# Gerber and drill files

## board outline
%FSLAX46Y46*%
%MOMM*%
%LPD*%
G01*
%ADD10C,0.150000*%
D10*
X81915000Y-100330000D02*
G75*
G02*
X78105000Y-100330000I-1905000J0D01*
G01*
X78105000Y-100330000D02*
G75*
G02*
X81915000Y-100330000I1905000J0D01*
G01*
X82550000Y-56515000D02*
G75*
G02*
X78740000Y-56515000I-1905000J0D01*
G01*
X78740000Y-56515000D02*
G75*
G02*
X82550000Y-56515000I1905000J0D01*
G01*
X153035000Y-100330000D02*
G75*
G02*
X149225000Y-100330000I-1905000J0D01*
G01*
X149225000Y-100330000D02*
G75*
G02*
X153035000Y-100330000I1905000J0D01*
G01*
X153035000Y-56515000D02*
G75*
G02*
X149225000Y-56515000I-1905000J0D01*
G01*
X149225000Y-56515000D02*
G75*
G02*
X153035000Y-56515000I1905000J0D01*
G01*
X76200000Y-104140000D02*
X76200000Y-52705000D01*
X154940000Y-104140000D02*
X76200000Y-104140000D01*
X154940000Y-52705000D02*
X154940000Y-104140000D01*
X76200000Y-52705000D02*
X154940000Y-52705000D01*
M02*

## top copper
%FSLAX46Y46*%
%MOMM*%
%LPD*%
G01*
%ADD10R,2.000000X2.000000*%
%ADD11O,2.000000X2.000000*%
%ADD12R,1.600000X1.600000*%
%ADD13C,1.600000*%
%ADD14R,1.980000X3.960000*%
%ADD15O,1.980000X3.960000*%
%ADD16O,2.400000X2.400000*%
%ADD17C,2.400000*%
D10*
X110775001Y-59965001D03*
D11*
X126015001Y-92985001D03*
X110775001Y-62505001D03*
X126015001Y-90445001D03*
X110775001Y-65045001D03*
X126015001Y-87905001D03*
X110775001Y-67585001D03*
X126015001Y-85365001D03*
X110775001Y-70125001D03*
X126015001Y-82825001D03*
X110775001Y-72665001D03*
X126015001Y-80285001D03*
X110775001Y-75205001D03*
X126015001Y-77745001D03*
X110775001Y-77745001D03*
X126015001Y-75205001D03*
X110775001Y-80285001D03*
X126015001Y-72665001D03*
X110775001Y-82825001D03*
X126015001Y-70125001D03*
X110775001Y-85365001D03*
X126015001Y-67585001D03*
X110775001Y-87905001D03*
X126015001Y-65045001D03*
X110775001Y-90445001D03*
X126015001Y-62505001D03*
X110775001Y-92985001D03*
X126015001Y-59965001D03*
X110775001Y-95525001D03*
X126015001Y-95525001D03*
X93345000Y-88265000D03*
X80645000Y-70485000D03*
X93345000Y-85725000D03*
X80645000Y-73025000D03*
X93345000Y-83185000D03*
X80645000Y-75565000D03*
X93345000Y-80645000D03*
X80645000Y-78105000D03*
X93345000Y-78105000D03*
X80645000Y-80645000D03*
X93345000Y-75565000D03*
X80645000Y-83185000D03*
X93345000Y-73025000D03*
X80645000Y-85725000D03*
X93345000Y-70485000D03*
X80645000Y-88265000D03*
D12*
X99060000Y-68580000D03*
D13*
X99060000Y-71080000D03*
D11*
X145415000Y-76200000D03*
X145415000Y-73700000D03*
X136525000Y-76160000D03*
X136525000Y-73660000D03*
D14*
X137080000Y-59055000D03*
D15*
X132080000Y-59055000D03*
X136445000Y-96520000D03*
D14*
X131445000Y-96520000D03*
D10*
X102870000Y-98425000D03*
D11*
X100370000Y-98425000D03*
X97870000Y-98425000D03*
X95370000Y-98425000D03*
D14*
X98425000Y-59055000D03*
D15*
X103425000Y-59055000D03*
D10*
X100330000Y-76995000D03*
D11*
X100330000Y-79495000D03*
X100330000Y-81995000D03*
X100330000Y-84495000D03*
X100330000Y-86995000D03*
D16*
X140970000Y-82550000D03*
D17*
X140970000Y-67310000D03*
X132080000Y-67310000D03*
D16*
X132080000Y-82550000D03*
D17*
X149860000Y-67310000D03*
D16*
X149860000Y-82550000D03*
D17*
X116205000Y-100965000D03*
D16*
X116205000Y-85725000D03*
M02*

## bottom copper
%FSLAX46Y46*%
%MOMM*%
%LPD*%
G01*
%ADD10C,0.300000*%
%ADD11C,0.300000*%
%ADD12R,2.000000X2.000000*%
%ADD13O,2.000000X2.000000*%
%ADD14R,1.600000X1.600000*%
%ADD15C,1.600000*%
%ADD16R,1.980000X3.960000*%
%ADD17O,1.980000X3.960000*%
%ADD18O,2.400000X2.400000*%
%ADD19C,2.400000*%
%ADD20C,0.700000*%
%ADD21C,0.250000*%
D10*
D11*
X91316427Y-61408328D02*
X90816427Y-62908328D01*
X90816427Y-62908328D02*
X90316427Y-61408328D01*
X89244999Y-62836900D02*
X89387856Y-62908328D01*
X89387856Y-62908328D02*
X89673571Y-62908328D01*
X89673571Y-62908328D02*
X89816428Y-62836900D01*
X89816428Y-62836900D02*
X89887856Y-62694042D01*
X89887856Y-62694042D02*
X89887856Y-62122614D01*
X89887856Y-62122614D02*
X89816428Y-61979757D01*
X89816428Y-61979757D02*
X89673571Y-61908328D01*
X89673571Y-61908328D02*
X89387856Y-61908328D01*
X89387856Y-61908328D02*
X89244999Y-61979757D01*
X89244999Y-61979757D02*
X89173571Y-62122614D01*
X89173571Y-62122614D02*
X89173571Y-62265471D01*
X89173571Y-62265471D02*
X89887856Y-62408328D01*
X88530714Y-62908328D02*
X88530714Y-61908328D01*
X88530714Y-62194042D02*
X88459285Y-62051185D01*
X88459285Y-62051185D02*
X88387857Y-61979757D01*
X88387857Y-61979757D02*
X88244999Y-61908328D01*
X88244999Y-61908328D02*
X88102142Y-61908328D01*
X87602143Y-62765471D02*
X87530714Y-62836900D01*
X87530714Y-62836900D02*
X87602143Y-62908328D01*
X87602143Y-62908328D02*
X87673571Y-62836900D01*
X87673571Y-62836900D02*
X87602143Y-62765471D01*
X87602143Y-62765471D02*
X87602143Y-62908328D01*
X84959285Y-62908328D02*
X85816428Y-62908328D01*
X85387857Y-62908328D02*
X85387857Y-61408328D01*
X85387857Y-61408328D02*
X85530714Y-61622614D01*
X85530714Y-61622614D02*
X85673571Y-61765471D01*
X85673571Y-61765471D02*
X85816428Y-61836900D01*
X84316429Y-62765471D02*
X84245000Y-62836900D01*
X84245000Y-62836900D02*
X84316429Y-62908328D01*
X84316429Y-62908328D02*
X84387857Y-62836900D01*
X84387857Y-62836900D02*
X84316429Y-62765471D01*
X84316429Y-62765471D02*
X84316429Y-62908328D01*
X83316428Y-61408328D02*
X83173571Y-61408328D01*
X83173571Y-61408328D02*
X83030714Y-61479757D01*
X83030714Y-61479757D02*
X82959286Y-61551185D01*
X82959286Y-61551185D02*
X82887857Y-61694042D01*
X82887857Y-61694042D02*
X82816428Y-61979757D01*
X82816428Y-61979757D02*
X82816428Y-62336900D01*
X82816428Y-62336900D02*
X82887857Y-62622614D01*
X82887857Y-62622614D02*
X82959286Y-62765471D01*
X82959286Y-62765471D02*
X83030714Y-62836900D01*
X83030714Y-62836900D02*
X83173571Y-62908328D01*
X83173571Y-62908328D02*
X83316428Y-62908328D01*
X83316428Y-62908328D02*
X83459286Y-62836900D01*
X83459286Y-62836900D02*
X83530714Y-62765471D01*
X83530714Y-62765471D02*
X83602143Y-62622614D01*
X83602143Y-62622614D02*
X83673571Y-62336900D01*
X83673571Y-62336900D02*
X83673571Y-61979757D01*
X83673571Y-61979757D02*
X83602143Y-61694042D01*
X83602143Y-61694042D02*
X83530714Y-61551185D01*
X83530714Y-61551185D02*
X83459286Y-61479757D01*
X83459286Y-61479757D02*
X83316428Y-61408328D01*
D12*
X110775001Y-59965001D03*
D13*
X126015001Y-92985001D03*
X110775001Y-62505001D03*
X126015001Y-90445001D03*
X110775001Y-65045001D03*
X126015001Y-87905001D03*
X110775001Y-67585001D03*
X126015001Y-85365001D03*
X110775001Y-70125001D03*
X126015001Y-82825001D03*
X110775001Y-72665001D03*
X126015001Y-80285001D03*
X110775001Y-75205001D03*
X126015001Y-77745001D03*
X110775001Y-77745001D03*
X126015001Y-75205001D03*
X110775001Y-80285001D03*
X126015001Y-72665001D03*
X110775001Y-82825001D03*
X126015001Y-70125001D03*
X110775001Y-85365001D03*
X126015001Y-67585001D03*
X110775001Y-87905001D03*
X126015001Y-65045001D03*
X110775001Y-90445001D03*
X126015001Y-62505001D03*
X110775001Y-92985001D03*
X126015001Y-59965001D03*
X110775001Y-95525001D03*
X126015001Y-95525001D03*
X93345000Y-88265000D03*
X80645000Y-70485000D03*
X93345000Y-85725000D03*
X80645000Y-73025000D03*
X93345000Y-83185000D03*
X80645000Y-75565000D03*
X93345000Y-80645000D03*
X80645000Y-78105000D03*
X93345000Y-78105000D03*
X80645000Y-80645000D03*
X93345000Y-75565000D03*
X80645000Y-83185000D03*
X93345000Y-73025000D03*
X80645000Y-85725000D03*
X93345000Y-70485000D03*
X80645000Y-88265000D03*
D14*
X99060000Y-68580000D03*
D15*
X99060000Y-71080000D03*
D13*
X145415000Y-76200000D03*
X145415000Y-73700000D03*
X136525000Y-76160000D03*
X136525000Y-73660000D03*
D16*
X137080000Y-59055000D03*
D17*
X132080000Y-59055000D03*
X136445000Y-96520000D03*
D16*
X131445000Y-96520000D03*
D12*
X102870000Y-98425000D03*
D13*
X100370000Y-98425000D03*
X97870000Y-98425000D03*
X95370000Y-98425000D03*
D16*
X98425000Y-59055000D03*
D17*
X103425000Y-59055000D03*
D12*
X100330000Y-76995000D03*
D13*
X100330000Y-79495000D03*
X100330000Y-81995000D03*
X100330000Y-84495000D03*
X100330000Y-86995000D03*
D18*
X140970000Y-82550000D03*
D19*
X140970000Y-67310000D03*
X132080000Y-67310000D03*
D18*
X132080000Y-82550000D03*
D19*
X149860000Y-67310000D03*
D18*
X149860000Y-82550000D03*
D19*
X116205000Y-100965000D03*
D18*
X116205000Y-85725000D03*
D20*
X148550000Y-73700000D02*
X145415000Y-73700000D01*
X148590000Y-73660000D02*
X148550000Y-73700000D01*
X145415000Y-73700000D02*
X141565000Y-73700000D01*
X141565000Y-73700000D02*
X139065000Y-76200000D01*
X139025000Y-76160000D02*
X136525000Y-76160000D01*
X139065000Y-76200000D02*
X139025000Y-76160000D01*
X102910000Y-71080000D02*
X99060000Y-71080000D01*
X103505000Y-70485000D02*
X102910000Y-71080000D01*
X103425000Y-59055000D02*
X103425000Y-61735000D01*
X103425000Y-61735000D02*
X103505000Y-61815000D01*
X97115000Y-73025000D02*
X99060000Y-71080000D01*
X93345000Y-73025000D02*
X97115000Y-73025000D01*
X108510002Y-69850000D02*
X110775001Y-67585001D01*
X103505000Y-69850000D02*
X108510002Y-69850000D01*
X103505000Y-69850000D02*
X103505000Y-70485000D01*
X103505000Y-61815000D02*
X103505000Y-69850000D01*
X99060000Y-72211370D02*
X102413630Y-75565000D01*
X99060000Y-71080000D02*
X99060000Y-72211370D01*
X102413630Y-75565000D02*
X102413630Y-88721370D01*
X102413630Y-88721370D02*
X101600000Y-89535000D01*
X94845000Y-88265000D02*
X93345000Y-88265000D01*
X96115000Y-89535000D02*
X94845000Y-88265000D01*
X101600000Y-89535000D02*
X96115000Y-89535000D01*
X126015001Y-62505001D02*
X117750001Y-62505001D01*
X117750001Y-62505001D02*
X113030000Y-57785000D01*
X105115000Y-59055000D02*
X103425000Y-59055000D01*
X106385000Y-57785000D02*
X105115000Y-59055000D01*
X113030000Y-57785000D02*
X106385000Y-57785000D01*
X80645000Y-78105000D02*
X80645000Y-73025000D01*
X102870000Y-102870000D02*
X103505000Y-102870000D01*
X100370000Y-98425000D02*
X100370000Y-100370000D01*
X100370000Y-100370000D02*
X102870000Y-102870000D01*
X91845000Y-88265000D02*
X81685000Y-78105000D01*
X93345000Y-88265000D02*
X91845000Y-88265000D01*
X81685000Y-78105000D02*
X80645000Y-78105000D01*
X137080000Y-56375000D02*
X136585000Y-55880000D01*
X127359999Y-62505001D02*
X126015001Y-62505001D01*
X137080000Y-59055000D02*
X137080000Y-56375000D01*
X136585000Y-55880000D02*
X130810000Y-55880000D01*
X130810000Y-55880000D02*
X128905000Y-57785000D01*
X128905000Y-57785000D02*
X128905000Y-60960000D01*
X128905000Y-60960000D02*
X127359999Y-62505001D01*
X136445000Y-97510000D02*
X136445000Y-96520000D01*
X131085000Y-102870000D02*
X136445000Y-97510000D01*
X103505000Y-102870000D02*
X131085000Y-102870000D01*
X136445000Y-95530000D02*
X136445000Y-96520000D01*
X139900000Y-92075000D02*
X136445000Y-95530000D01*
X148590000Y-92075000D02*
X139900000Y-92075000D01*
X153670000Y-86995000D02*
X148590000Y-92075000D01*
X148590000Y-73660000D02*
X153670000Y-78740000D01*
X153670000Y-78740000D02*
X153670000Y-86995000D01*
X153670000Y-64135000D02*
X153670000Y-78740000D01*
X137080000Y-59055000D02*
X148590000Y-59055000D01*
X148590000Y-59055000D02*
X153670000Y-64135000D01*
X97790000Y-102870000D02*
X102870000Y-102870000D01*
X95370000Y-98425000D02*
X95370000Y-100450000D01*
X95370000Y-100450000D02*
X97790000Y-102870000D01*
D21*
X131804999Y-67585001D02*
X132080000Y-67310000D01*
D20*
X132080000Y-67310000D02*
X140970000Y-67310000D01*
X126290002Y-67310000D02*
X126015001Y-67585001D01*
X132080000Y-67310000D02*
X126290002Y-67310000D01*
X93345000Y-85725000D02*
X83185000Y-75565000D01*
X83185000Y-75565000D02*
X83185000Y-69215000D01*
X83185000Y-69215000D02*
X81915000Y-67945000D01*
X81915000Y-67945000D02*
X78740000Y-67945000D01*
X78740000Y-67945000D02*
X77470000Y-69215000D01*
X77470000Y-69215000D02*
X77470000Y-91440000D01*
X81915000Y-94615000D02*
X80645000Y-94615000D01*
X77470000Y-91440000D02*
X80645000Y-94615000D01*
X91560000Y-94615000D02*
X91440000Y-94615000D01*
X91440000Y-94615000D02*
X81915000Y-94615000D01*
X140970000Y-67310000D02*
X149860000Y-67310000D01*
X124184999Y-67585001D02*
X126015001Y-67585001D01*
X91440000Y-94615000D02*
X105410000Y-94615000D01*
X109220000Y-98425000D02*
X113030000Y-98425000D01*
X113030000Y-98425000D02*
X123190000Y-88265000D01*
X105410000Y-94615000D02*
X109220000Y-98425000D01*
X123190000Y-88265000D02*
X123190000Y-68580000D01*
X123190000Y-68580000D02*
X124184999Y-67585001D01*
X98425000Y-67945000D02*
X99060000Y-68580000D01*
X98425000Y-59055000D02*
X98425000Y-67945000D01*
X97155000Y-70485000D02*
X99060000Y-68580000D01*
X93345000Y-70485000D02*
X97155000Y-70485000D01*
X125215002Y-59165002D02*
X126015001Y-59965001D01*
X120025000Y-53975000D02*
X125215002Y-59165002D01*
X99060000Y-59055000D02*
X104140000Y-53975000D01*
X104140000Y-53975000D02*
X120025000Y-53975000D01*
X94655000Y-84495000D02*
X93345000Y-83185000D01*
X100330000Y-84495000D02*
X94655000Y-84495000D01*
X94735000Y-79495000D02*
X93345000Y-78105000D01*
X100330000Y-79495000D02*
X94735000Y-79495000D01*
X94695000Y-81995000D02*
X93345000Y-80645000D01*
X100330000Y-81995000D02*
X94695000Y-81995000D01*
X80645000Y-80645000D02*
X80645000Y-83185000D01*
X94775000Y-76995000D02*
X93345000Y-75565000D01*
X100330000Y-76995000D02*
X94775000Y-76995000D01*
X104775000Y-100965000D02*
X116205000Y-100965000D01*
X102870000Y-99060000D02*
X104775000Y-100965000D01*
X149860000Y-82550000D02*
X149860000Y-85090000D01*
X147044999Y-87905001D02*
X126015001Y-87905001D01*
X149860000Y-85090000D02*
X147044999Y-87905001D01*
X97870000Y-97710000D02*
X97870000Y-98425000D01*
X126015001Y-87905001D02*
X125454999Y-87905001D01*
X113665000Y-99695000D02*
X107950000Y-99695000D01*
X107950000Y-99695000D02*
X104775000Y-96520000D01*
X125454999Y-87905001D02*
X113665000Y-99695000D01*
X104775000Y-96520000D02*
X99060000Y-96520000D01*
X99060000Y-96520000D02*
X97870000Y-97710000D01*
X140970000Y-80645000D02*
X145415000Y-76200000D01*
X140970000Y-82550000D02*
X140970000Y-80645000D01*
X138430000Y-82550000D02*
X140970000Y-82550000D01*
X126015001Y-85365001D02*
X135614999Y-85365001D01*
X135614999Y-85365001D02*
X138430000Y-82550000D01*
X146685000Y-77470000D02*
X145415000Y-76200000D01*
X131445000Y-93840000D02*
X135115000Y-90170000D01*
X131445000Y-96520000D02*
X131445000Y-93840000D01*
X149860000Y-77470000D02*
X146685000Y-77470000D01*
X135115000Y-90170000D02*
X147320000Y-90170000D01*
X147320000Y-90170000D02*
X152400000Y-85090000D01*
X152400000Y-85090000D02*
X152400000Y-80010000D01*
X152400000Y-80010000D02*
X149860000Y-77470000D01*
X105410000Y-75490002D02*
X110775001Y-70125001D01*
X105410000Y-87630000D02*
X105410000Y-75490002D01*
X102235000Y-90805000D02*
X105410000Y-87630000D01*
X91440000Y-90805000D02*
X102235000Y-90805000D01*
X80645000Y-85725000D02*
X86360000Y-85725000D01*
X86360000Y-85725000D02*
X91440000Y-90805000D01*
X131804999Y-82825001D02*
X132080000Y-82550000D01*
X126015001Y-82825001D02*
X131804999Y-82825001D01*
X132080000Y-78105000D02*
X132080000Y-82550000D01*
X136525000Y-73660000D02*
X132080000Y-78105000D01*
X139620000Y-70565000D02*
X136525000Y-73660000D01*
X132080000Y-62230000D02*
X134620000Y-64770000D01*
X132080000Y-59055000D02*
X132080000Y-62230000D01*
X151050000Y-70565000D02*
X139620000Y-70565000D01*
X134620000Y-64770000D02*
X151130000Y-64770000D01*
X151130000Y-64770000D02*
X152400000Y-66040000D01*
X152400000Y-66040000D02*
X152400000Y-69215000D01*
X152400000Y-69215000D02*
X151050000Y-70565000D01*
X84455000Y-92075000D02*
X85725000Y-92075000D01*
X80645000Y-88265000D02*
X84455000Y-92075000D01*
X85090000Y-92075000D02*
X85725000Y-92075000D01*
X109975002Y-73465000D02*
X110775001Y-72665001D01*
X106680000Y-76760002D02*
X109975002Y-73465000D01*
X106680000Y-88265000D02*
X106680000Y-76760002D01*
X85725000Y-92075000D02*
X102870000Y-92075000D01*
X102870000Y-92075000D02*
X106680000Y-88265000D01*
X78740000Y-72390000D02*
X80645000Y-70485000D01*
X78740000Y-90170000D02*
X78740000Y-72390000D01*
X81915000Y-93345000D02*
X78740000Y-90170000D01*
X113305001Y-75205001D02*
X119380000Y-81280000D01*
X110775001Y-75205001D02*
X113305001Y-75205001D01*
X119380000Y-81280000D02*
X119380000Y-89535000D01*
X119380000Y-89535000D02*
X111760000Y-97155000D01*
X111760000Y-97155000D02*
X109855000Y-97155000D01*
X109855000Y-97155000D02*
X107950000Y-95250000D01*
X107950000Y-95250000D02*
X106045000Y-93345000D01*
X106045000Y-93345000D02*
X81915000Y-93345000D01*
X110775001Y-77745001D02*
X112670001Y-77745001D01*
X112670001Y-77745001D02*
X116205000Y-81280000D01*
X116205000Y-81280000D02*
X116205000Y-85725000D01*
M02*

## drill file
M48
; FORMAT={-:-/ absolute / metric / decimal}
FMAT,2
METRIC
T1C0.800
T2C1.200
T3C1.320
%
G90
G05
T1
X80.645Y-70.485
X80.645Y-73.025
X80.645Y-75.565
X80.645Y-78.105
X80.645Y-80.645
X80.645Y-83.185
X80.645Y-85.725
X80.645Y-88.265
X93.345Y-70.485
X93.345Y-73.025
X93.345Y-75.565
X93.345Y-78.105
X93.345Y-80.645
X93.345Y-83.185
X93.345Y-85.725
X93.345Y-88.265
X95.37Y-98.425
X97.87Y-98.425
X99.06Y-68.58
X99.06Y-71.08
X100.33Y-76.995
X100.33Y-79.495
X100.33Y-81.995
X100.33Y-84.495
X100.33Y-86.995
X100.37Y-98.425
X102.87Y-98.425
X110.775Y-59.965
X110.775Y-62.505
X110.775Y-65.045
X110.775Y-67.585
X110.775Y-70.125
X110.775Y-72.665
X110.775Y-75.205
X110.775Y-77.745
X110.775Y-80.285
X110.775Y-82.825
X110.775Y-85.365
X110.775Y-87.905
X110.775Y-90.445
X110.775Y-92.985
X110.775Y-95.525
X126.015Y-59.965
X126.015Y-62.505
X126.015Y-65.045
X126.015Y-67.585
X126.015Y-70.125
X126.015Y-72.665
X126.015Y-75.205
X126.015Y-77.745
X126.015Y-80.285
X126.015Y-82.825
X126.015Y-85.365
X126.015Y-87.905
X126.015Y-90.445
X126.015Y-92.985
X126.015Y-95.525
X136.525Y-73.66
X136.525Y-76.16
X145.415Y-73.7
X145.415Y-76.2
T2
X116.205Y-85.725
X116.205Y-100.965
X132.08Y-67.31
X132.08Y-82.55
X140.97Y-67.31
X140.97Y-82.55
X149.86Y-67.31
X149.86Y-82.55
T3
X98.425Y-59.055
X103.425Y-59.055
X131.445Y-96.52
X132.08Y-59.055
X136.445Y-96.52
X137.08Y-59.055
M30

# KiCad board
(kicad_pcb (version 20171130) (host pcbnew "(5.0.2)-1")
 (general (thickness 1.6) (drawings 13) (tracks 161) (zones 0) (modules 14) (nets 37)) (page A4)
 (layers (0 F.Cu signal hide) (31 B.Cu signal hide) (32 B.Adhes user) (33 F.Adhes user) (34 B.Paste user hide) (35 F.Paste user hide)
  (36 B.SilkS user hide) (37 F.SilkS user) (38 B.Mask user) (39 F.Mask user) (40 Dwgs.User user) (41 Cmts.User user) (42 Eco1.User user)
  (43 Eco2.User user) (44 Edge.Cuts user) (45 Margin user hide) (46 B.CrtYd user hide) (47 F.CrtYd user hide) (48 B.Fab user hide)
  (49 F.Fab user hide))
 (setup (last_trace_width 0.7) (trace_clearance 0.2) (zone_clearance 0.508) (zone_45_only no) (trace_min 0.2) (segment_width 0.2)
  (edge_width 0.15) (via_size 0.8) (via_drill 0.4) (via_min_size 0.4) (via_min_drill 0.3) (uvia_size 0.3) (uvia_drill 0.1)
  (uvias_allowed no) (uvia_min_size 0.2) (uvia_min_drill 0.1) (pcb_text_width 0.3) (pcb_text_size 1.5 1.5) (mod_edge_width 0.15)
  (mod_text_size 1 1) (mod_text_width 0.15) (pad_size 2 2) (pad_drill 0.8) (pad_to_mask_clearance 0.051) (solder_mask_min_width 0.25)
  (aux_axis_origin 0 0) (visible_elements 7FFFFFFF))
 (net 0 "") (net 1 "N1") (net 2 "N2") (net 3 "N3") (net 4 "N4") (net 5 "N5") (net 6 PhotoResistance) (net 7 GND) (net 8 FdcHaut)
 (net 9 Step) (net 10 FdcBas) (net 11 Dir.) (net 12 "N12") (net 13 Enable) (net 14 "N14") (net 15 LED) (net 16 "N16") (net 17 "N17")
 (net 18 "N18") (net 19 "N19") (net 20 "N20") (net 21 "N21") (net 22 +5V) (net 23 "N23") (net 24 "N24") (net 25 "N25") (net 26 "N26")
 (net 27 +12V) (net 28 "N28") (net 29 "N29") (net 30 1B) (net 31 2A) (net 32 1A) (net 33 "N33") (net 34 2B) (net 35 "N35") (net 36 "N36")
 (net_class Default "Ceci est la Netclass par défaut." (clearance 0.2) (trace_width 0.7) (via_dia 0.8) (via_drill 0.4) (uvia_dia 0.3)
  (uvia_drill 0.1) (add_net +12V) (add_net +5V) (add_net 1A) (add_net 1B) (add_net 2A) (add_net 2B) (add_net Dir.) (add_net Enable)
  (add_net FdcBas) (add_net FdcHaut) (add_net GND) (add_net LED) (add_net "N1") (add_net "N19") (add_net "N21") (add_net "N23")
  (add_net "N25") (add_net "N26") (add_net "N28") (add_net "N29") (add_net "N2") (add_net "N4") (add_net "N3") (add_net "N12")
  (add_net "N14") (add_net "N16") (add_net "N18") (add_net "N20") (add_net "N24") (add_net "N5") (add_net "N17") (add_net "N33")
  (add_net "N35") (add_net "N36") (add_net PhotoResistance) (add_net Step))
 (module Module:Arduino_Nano (layer F.Cu) (at 110.775001 59.965001)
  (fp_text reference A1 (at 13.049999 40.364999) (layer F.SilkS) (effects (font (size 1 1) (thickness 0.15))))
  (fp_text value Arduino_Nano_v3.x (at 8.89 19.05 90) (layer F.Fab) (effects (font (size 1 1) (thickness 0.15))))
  (pad 1 thru_hole rect (at 0 0) (size 2 2) (drill 0.8) (layers *.Cu *.Mask) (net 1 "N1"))
  (pad 17 thru_hole oval (at 15.24 33.02) (size 2 2) (drill 0.8) (layers *.Cu *.Mask) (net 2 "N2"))
  (pad 2 thru_hole oval (at 0 2.54) (size 2 2) (drill 0.8) (layers *.Cu *.Mask) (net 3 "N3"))
  (pad 18 thru_hole oval (at 15.24 30.48) (size 2 2) (drill 0.8) (layers *.Cu *.Mask) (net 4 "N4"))
  (pad 3 thru_hole oval (at 0 5.08) (size 2 2) (drill 0.8) (layers *.Cu *.Mask) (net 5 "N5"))
  (pad 19 thru_hole oval (at 15.24 27.94) (size 2 2) (drill 0.8) (layers *.Cu *.Mask) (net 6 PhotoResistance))
  (pad 4 thru_hole oval (at 0 7.62) (size 2 2) (drill 0.8) (layers *.Cu *.Mask) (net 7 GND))
  (pad 20 thru_hole oval (at 15.24 25.4) (size 2 2) (drill 0.8) (layers *.Cu *.Mask) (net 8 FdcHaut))
  (pad 5 thru_hole oval (at 0 10.16) (size 2 2) (drill 0.8) (layers *.Cu *.Mask) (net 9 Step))
  (pad 21 thru_hole oval (at 15.24 22.86) (size 2 2) (drill 0.8) (layers *.Cu *.Mask) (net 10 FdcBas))
  (pad 6 thru_hole oval (at 0 12.7) (size 2 2) (drill 0.8) (layers *.Cu *.Mask) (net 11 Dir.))
  (pad 22 thru_hole oval (at 15.24 20.32) (size 2 2) (drill 0.8) (layers *.Cu *.Mask) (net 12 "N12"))
  (pad 7 thru_hole oval (at 0 15.24) (size 2 2) (drill 0.8) (layers *.Cu *.Mask) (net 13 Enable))
  (pad 23 thru_hole oval (at 15.24 17.78) (size 2 2) (drill 0.8) (layers *.Cu *.Mask) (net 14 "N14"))
  (pad 8 thru_hole oval (at 0 17.78) (size 2 2) (drill 0.8) (layers *.Cu *.Mask) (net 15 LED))
  (pad 24 thru_hole oval (at 15.24 15.24) (size 2 2) (drill 0.8) (layers *.Cu *.Mask) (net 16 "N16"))
  (pad 9 thru_hole oval (at 0 20.32) (size 2 2) (drill 0.8) (layers *.Cu *.Mask) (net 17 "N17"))
  (pad 25 thru_hole oval (at 15.24 12.7) (size 2 2) (drill 0.8) (layers *.Cu *.Mask) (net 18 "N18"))
  (pad 10 thru_hole oval (at 0 22.86) (size 2 2) (drill 0.8) (layers *.Cu *.Mask) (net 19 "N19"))
  (pad 26 thru_hole oval (at 15.24 10.16) (size 2 2) (drill 0.8) (layers *.Cu *.Mask) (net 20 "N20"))
  (pad 11 thru_hole oval (at 0 25.4) (size 2 2) (drill 0.8) (layers *.Cu *.Mask) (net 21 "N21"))
  (pad 27 thru_hole oval (at 15.24 7.62) (size 2 2) (drill 0.8) (layers *.Cu *.Mask) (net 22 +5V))
  (pad 12 thru_hole oval (at 0 27.94) (size 2 2) (drill 0.8) (layers *.Cu *.Mask) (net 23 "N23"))
  (pad 28 thru_hole oval (at 15.24 5.08) (size 2 2) (drill 0.8) (layers *.Cu *.Mask) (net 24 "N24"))
  (pad 13 thru_hole oval (at 0 30.48) (size 2 2) (drill 0.8) (layers *.Cu *.Mask) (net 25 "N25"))
  (pad 29 thru_hole oval (at 15.24 2.54) (size 2 2) (drill 0.8) (layers *.Cu *.Mask) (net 7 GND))
  (pad 14 thru_hole oval (at 0 33.02) (size 2 2) (drill 0.8) (layers *.Cu *.Mask) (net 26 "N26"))
  (pad 30 thru_hole oval (at 15.24 0) (size 2 2) (drill 0.8) (layers *.Cu *.Mask) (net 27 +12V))
  (pad 15 thru_hole oval (at 0 35.56) (size 2 2) (drill 0.8) (layers *.Cu *.Mask) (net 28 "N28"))
  (pad 16 thru_hole oval (at 15.24 35.56) (size 2 2) (drill 0.8) (layers *.Cu *.Mask) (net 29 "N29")))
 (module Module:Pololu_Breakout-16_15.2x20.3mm (layer F.Cu) (at 93.345 88.265 180)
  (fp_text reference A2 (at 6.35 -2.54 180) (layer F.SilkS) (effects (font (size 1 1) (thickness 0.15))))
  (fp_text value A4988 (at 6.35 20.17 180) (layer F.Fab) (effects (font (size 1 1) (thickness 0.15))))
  (pad 1 thru_hole oval (at 0 0 180) (size 2 2) (drill 0.8) (layers *.Cu *.Mask) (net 7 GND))
  (pad 9 thru_hole oval (at 12.7 17.78 180) (size 2 2) (drill 0.8) (layers *.Cu *.Mask) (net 13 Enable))
  (pad 2 thru_hole oval (at 0 2.54 180) (size 2 2) (drill 0.8) (layers *.Cu *.Mask) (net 22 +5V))
  (pad 10 thru_hole oval (at 12.7 15.24 180) (size 2 2) (drill 0.8) (layers *.Cu *.Mask) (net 7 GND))
  (pad 3 thru_hole oval (at 0 5.08 180) (size 2 2) (drill 0.8) (layers *.Cu *.Mask) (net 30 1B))
  (pad 11 thru_hole oval (at 12.7 12.7 180) (size 2 2) (drill 0.8) (layers *.Cu *.Mask) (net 7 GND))
  (pad 4 thru_hole oval (at 0 7.62 180) (size 2 2) (drill 0.8) (layers *.Cu *.Mask) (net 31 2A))
  (pad 12 thru_hole oval (at 12.7 10.16 180) (size 2 2) (drill 0.8) (layers *.Cu *.Mask) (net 7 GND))
  (pad 5 thru_hole oval (at 0 10.16 180) (size 2 2) (drill 0.8) (layers *.Cu *.Mask) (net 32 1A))
  (pad 13 thru_hole oval (at 12.7 7.62 180) (size 2 2) (drill 0.8) (layers *.Cu *.Mask) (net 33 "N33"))
  (pad 6 thru_hole oval (at 0 12.7 180) (size 2 2) (drill 0.8) (layers *.Cu *.Mask) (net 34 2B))
  (pad 14 thru_hole oval (at 12.7 5.08 180) (size 2 2) (drill 0.8) (layers *.Cu *.Mask) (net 33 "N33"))
  (pad 7 thru_hole oval (at 0 15.24 180) (size 2 2) (drill 0.8) (layers *.Cu *.Mask) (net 7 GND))
  (pad 15 thru_hole oval (at 12.7 2.54 180) (size 2 2) (drill 0.8) (layers *.Cu *.Mask) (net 9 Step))
  (pad 8 thru_hole oval (at 0 17.78 180) (size 2 2) (drill 0.8) (layers *.Cu *.Mask) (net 27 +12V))
  (pad 16 thru_hole oval (at 12.7 0 180) (size 2 2) (drill 0.8) (layers *.Cu *.Mask) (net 11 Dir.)))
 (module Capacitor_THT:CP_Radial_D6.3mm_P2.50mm (layer F.Cu) (at 99.06 68.58 270)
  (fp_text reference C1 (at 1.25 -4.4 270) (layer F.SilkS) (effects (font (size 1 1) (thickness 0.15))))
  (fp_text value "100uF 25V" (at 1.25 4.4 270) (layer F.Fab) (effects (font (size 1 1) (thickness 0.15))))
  (pad 1 thru_hole rect (at 0 0 270) (size 1.6 1.6) (drill 0.8) (layers *.Cu *.Mask) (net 27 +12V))
  (pad 2 thru_hole circle (at 2.5 0 270) (size 1.6 1.6) (drill 0.8) (layers *.Cu *.Mask) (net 7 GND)))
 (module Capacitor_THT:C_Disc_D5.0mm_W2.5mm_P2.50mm (layer F.Cu) (at 145.415 76.2 90)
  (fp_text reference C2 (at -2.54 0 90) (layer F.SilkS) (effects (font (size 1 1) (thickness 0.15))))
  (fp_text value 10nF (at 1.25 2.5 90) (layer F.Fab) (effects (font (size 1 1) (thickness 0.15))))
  (pad 1 thru_hole oval (at 0 0 90) (size 2 2) (drill 0.8) (layers *.Cu *.Mask) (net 8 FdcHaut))
  (pad 2 thru_hole oval (at 2.5 0 90) (size 2 2) (drill 0.8) (layers *.Cu *.Mask) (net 7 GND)))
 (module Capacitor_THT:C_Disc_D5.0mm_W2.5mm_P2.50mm (layer F.Cu) (at 136.525 73.66 270)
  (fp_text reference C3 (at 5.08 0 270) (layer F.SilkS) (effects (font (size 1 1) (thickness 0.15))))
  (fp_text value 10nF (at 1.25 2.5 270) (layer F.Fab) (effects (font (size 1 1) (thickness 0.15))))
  (pad 2 thru_hole oval (at 2.5 0 270) (size 2 2) (drill 0.8) (layers *.Cu *.Mask) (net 7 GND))
  (pad 1 thru_hole oval (at 0 0 270) (size 2 2) (drill 0.8) (layers *.Cu *.Mask) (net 10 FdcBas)))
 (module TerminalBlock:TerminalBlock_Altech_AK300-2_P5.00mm (layer F.Cu) (at 137.08 59.055 180)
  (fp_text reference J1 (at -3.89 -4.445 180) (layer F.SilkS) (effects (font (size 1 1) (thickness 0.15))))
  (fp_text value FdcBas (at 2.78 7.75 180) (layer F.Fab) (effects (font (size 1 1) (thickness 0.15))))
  (pad 1 thru_hole rect (at 0 0 180) (size 1.98 3.96) (drill 1.32) (layers *.Cu *.Mask) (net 7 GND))
  (pad 2 thru_hole oval (at 5 0 180) (size 1.98 3.96) (drill 1.32) (layers *.Cu *.Mask) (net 10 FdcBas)))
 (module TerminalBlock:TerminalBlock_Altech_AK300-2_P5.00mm (layer F.Cu) (at 131.445 96.52)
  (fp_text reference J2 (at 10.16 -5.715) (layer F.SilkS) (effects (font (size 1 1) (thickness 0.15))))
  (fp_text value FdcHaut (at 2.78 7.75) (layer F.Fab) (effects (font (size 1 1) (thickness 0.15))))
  (pad 2 thru_hole oval (at 5 0) (size 1.98 3.96) (drill 1.32) (layers *.Cu *.Mask) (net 7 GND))
  (pad 1 thru_hole rect (at 0 0) (size 1.98 3.96) (drill 1.32) (layers *.Cu *.Mask) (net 8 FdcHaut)))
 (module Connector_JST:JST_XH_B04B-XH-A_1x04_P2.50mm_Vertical (layer F.Cu) (at 102.87 98.425 180)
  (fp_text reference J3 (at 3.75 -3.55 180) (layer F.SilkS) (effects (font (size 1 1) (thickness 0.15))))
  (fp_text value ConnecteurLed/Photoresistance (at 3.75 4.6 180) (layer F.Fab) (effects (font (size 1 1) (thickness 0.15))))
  (pad 1 thru_hole rect (at 0 0 180) (size 2 2) (drill 0.8) (layers *.Cu *.Mask) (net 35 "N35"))
  (pad 2 thru_hole oval (at 2.5 0 180) (size 2 2) (drill 0.8) (layers *.Cu *.Mask) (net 7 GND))
  (pad 3 thru_hole oval (at 5 0 180) (size 2 2) (drill 0.8) (layers *.Cu *.Mask) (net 6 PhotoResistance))
  (pad 4 thru_hole oval (at 7.5 0 180) (size 2 2) (drill 0.8) (layers *.Cu *.Mask) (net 7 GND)))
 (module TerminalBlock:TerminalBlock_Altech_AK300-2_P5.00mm (layer F.Cu) (at 98.425 59.055)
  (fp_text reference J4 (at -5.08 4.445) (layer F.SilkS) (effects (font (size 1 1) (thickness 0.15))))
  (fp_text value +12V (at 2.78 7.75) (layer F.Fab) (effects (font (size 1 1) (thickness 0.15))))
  (pad 1 thru_hole rect (at 0 0) (size 1.98 3.96) (drill 1.32) (layers *.Cu *.Mask) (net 27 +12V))
  (pad 2 thru_hole oval (at 5 0) (size 1.98 3.96) (drill 1.32) (layers *.Cu *.Mask) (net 7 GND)))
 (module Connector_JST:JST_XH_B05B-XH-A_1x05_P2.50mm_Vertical (layer F.Cu) (at 100.33 76.995 270)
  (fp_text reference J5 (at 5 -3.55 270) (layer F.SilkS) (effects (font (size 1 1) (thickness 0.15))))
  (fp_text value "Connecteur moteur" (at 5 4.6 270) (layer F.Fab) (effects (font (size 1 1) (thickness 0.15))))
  (pad 1 thru_hole rect (at 0 0 270) (size 2 2) (drill 0.8) (layers *.Cu *.Mask) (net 34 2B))
  (pad 2 thru_hole oval (at 2.5 0 270) (size 2 2) (drill 0.8) (layers *.Cu *.Mask) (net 32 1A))
  (pad 3 thru_hole oval (at 5 0 270) (size 2 2) (drill 0.8) (layers *.Cu *.Mask) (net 31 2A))
  (pad 4 thru_hole oval (at 7.5 0 270) (size 2 2) (drill 0.8) (layers *.Cu *.Mask) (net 30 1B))
  (pad 5 thru_hole oval (at 10 0 270) (size 2 2) (drill 0.8) (layers *.Cu *.Mask) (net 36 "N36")))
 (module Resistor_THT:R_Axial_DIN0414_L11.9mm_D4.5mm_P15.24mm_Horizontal (layer F.Cu) (at 140.97 67.31 270)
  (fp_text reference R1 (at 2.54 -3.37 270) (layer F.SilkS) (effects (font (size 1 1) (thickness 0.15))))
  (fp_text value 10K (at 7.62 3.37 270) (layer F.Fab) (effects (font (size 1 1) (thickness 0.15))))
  (pad 2 thru_hole oval (at 15.24 0 270) (size 2.4 2.4) (drill 1.2) (layers *.Cu *.Mask) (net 8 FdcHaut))
  (pad 1 thru_hole circle (at 0 0 270) (size 2.4 2.4) (drill 1.2) (layers *.Cu *.Mask) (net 22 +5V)))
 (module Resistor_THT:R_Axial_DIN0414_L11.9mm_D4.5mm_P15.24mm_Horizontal (layer F.Cu) (at 132.08 67.31 270)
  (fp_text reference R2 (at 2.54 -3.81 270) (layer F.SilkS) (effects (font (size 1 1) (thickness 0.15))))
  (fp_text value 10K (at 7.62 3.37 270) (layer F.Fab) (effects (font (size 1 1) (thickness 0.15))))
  (pad 1 thru_hole circle (at 0 0 270) (size 2.4 2.4) (drill 1.2) (layers *.Cu *.Mask) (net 22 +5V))
  (pad 2 thru_hole oval (at 15.24 0 270) (size 2.4 2.4) (drill 1.2) (layers *.Cu *.Mask) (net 10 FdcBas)))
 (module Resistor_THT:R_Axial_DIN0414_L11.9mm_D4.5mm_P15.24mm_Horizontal (layer F.Cu) (at 149.86 67.31 270)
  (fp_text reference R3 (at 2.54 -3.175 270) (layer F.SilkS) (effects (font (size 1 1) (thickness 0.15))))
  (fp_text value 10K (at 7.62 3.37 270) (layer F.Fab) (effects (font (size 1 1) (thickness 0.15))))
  (pad 1 thru_hole circle (at 0 0 270) (size 2.4 2.4) (drill 1.2) (layers *.Cu *.Mask) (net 22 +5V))
  (pad 2 thru_hole oval (at 15.24 0 270) (size 2.4 2.4) (drill 1.2) (layers *.Cu *.Mask) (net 6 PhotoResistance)))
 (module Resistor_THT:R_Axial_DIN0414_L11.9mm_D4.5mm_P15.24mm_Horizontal (layer F.Cu) (at 116.205 100.965 90)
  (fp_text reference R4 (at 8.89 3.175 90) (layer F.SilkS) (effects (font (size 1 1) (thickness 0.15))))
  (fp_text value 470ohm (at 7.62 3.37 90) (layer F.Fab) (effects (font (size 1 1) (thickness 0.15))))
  (pad 1 thru_hole circle (at 0 0 90) (size 2.4 2.4) (drill 1.2) (layers *.Cu *.Mask) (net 35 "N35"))
  (pad 2 thru_hole oval (at 15.24 0 90) (size 2.4 2.4) (drill 1.2) (layers *.Cu *.Mask) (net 15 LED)))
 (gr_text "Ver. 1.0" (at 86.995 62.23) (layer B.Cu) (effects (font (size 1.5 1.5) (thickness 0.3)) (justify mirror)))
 (gr_circle (center 80.01 100.33) (end 81.915 100.33) (layer Edge.Cuts) (width 0.15))
 (gr_circle (center 80.645 56.515) (end 82.55 56.515) (layer Edge.Cuts) (width 0.15))
 (gr_circle (center 151.13 100.33) (end 151.13 98.425) (layer Edge.Cuts) (width 0.15))
 (gr_circle (center 151.13 56.515) (end 151.13 54.61) (layer Edge.Cuts) (width 0.15))
 (gr_line (start 76.2 104.14) (end 76.2 52.705) (layer Edge.Cuts) (width 0.15))
 (gr_line (start 154.94 104.14) (end 76.2 104.14) (layer Edge.Cuts) (width 0.15))
 (gr_line (start 154.94 52.705) (end 154.94 104.14) (layer Edge.Cuts) (width 0.15))
 (gr_line (start 76.2 52.705) (end 154.94 52.705) (layer Edge.Cuts) (width 0.15))
 (segment (start 148.55 73.7) (end 145.415 73.7) (width 0.7) (layer B.Cu) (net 7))
 (segment (start 148.59 73.66) (end 148.55 73.7) (width 0.7) (layer B.Cu) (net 7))
 (segment (start 145.415 73.7) (end 141.565 73.7) (width 0.7) (layer B.Cu) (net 7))
 (segment (start 141.565 73.7) (end 139.065 76.2) (width 0.7) (layer B.Cu) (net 7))
 (segment (start 139.025 76.16) (end 136.525 76.16) (width 0.7) (layer B.Cu) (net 7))
 (segment (start 139.065 76.2) (end 139.025 76.16) (width 0.7) (layer B.Cu) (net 7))
 (segment (start 102.91 71.08) (end 99.06 71.08) (width 0.7) (layer B.Cu) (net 7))
 (segment (start 103.505 70.485) (end 102.91 71.08) (width 0.7) (layer B.Cu) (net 7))
 (segment (start 103.425 59.055) (end 103.425 61.735) (width 0.7) (layer B.Cu) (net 7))
 (segment (start 103.425 61.735) (end 103.505 61.815) (width 0.7) (layer B.Cu) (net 7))
 (segment (start 97.115 73.025) (end 99.06 71.08) (width 0.7) (layer B.Cu) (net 7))
 (segment (start 93.345 73.025) (end 97.115 73.025) (width 0.7) (layer B.Cu) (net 7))
 (segment (start 108.510002 69.85) (end 110.775001 67.585001) (width 0.7) (layer B.Cu) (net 7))
 (segment (start 103.505 69.85) (end 108.510002 69.85) (width 0.7) (layer B.Cu) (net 7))
 (segment (start 103.505 69.85) (end 103.505 70.485) (width 0.7) (layer B.Cu) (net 7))
 (segment (start 103.505 61.815) (end 103.505 69.85) (width 0.7) (layer B.Cu) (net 7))
 (segment (start 99.06 72.21137) (end 102.41363 75.565) (width 0.7) (layer B.Cu) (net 7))
 (segment (start 99.06 71.08) (end 99.06 72.21137) (width 0.7) (layer B.Cu) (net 7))
 (segment (start 102.41363 75.565) (end 102.41363 88.72137) (width 0.7) (layer B.Cu) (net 7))
 (segment (start 102.41363 88.72137) (end 101.6 89.535) (width 0.7) (layer B.Cu) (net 7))
 (segment (start 94.845 88.265) (end 93.345 88.265) (width 0.7) (layer B.Cu) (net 7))
 (segment (start 96.115 89.535) (end 94.845 88.265) (width 0.7) (layer B.Cu) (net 7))
 (segment (start 101.6 89.535) (end 96.115 89.535) (width 0.7) (layer B.Cu) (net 7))
 (segment (start 126.015001 62.505001) (end 117.750001 62.505001) (width 0.7) (layer B.Cu) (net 7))
 (segment (start 117.750001 62.505001) (end 113.03 57.785) (width 0.7) (layer B.Cu) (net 7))
 (segment (start 105.115 59.055) (end 103.425 59.055) (width 0.7) (layer B.Cu) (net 7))
 (segment (start 106.385 57.785) (end 105.115 59.055) (width 0.7) (layer B.Cu) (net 7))
 (segment (start 113.03 57.785) (end 106.385 57.785) (width 0.7) (layer B.Cu) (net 7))
 (segment (start 80.645 78.105) (end 80.645 73.025) (width 0.7) (layer B.Cu) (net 7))
 (segment (start 102.87 102.87) (end 103.505 102.87) (width 0.7) (layer B.Cu) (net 7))
 (segment (start 100.37 98.425) (end 100.37 100.37) (width 0.7) (layer B.Cu) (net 7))
 (segment (start 100.37 100.37) (end 102.87 102.87) (width 0.7) (layer B.Cu) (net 7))
 (segment (start 91.845 88.265) (end 81.685 78.105) (width 0.7) (layer B.Cu) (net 7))
 (segment (start 93.345 88.265) (end 91.845 88.265) (width 0.7) (layer B.Cu) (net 7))
 (segment (start 81.685 78.105) (end 80.645 78.105) (width 0.7) (layer B.Cu) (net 7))
 (segment (start 137.08 56.375) (end 136.585 55.88) (width 0.7) (layer B.Cu) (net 7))
 (segment (start 127.359999 62.505001) (end 126.015001 62.505001) (width 0.7) (layer B.Cu) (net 7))
 (segment (start 137.08 59.055) (end 137.08 56.375) (width 0.7) (layer B.Cu) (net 7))
 (segment (start 136.585 55.88) (end 130.81 55.88) (width 0.7) (layer B.Cu) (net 7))
 (segment (start 130.81 55.88) (end 128.905 57.785) (width 0.7) (layer B.Cu) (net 7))
 (segment (start 128.905 57.785) (end 128.905 60.96) (width 0.7) (layer B.Cu) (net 7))
 (segment (start 128.905 60.96) (end 127.359999 62.505001) (width 0.7) (layer B.Cu) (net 7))
 (segment (start 136.445 97.51) (end 136.445 96.52) (width 0.7) (layer B.Cu) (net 7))
 (segment (start 131.085 102.87) (end 136.445 97.51) (width 0.7) (layer B.Cu) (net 7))
 (segment (start 103.505 102.87) (end 131.085 102.87) (width 0.7) (layer B.Cu) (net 7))
 (segment (start 136.445 95.53) (end 136.445 96.52) (width 0.7) (layer B.Cu) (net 7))
 (segment (start 139.9 92.075) (end 136.445 95.53) (width 0.7) (layer B.Cu) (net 7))
 (segment (start 148.59 92.075) (end 139.9 92.075) (width 0.7) (layer B.Cu) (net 7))
 (segment (start 153.67 86.995) (end 148.59 92.075) (width 0.7) (layer B.Cu) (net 7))
 (segment (start 148.59 73.66) (end 153.67 78.74) (width 0.7) (layer B.Cu) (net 7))
 (segment (start 153.67 78.74) (end 153.67 86.995) (width 0.7) (layer B.Cu) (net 7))
 (segment (start 153.67 64.135) (end 153.67 78.74) (width 0.7) (layer B.Cu) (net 7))
 (segment (start 137.08 59.055) (end 148.59 59.055) (width 0.7) (layer B.Cu) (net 7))
 (segment (start 148.59 59.055) (end 153.67 64.135) (width 0.7) (layer B.Cu) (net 7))
 (segment (start 97.79 102.87) (end 102.87 102.87) (width 0.7) (layer B.Cu) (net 7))
 (segment (start 95.37 98.425) (end 95.37 100.45) (width 0.7) (layer B.Cu) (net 7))
 (segment (start 95.37 100.45) (end 97.79 102.87) (width 0.7) (layer B.Cu) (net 7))
 (segment (start 131.804999 67.585001) (end 132.08 67.31) (width 0.25) (layer B.Cu) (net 22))
 (segment (start 132.08 67.31) (end 140.97 67.31) (width 0.7) (layer B.Cu) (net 22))
 (segment (start 126.290002 67.31) (end 126.015001 67.585001) (width 0.7) (layer B.Cu) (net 22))
 (segment (start 132.08 67.31) (end 126.290002 67.31) (width 0.7) (layer B.Cu) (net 22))
 (segment (start 93.345 85.725) (end 83.185 75.565) (width 0.7) (layer B.Cu) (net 22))
 (segment (start 83.185 75.565) (end 83.185 69.215) (width 0.7) (layer B.Cu) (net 22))
 (segment (start 83.185 69.215) (end 81.915 67.945) (width 0.7) (layer B.Cu) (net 22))
 (segment (start 81.915 67.945) (end 78.74 67.945) (width 0.7) (layer B.Cu) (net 22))
 (segment (start 78.74 67.945) (end 77.47 69.215) (width 0.7) (layer B.Cu) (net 22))
 (segment (start 77.47 69.215) (end 77.47 91.44) (width 0.7) (layer B.Cu) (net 22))
 (segment (start 81.915 94.615) (end 80.645 94.615) (width 0.7) (layer B.Cu) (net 22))
 (segment (start 77.47 91.44) (end 80.645 94.615) (width 0.7) (layer B.Cu) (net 22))
 (segment (start 91.56 94.615) (end 91.44 94.615) (width 0.7) (layer B.Cu) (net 22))
 (segment (start 91.44 94.615) (end 81.915 94.615) (width 0.7) (layer B.Cu) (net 22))
 (segment (start 140.97 67.31) (end 149.86 67.31) (width 0.7) (layer B.Cu) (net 22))
 (segment (start 124.184999 67.585001) (end 126.015001 67.585001) (width 0.7) (layer B.Cu) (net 22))
 (segment (start 91.44 94.615) (end 105.41 94.615) (width 0.7) (layer B.Cu) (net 22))
 (segment (start 109.22 98.425) (end 113.03 98.425) (width 0.7) (layer B.Cu) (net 22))
 (segment (start 113.03 98.425) (end 123.19 88.265) (width 0.7) (layer B.Cu) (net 22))
 (segment (start 105.41 94.615) (end 109.22 98.425) (width 0.7) (layer B.Cu) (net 22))
 (segment (start 123.19 88.265) (end 123.19 68.58) (width 0.7) (layer B.Cu) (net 22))
 (segment (start 123.19 68.58) (end 124.184999 67.585001) (width 0.7) (layer B.Cu) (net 22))
 (segment (start 98.425 67.945) (end 99.06 68.58) (width 0.7) (layer B.Cu) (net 27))
 (segment (start 98.425 59.055) (end 98.425 67.945) (width 0.7) (layer B.Cu) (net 27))
 (segment (start 97.155 70.485) (end 99.06 68.58) (width 0.7) (layer B.Cu) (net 27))
 (segment (start 93.345 70.485) (end 97.155 70.485) (width 0.7) (layer B.Cu) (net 27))
 (segment (start 125.215002 59.165002) (end 126.015001 59.965001) (width 0.7) (layer B.Cu) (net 27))
 (segment (start 120.025 53.975) (end 125.215002 59.165002) (width 0.7) (layer B.Cu) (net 27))
 (segment (start 99.06 59.055) (end 104.14 53.975) (width 0.7) (layer B.Cu) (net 27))
 (segment (start 104.14 53.975) (end 120.025 53.975) (width 0.7) (layer B.Cu) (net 27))
 (segment (start 94.655 84.495) (end 93.345 83.185) (width 0.7) (layer B.Cu) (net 30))
 (segment (start 100.33 84.495) (end 94.655 84.495) (width 0.7) (layer B.Cu) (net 30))
 (segment (start 94.735 79.495) (end 93.345 78.105) (width 0.7) (layer B.Cu) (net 32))
 (segment (start 100.33 79.495) (end 94.735 79.495) (width 0.7) (layer B.Cu) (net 32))
 (segment (start 94.695 81.995) (end 93.345 80.645) (width 0.7) (layer B.Cu) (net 31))
 (segment (start 100.33 81.995) (end 94.695 81.995) (width 0.7) (layer B.Cu) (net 31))
 (segment (start 80.645 80.645) (end 80.645 83.185) (width 0.7) (layer B.Cu) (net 33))
 (segment (start 94.775 76.995) (end 93.345 75.565) (width 0.7) (layer B.Cu) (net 34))
 (segment (start 100.33 76.995) (end 94.775 76.995) (width 0.7) (layer B.Cu) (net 34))
 (segment (start 104.775 100.965) (end 116.205 100.965) (width 0.7) (layer B.Cu) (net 35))
 (segment (start 102.87 99.06) (end 104.775 100.965) (width 0.7) (layer B.Cu) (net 35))
 (segment (start 149.86 82.55) (end 149.86 85.09) (width 0.7) (layer B.Cu) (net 6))
 (segment (start 147.044999 87.905001) (end 126.015001 87.905001) (width 0.7) (layer B.Cu) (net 6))
 (segment (start 149.86 85.09) (end 147.044999 87.905001) (width 0.7) (layer B.Cu) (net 6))
 (segment (start 97.87 97.71) (end 97.87 98.425) (width 0.7) (layer B.Cu) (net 6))
 (segment (start 126.015001 87.905001) (end 125.454999 87.905001) (width 0.7) (layer B.Cu) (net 6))
 (segment (start 113.665 99.695) (end 107.95 99.695) (width 0.7) (layer B.Cu) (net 6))
 (segment (start 107.95 99.695) (end 104.775 96.52) (width 0.7) (layer B.Cu) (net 6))
 (segment (start 125.454999 87.905001) (end 113.665 99.695) (width 0.7) (layer B.Cu) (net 6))
 (segment (start 104.775 96.52) (end 99.06 96.52) (width 0.7) (layer B.Cu) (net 6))
 (segment (start 99.06 96.52) (end 97.87 97.71) (width 0.7) (layer B.Cu) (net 6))
 (segment (start 140.97 80.645) (end 145.415 76.2) (width 0.7) (layer B.Cu) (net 8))
 (segment (start 140.97 82.55) (end 140.97 80.645) (width 0.7) (layer B.Cu) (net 8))
 (segment (start 138.43 82.55) (end 140.97 82.55) (width 0.7) (layer B.Cu) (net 8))
 (segment (start 126.015001 85.365001) (end 135.614999 85.365001) (width 0.7) (layer B.Cu) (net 8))
 (segment (start 135.614999 85.365001) (end 138.43 82.55) (width 0.7) (layer B.Cu) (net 8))
 (segment (start 146.685 77.47) (end 145.415 76.2) (width 0.7) (layer B.Cu) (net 8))
 (segment (start 131.445 93.84) (end 135.115 90.17) (width 0.7) (layer B.Cu) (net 8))
 (segment (start 131.445 96.52) (end 131.445 93.84) (width 0.7) (layer B.Cu) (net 8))
 (segment (start 149.86 77.47) (end 146.685 77.47) (width 0.7) (layer B.Cu) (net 8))
 (segment (start 135.115 90.17) (end 147.32 90.17) (width 0.7) (layer B.Cu) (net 8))
 (segment (start 147.32 90.17) (end 152.4 85.09) (width 0.7) (layer B.Cu) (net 8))
 (segment (start 152.4 85.09) (end 152.4 80.01) (width 0.7) (layer B.Cu) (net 8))
 (segment (start 152.4 80.01) (end 149.86 77.47) (width 0.7) (layer B.Cu) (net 8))
 (segment (start 105.41 75.490002) (end 110.775001 70.125001) (width 0.7) (layer B.Cu) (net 9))
 (segment (start 105.41 87.63) (end 105.41 75.490002) (width 0.7) (layer B.Cu) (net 9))
 (segment (start 102.235 90.805) (end 105.41 87.63) (width 0.7) (layer B.Cu) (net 9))
 (segment (start 91.44 90.805) (end 102.235 90.805) (width 0.7) (layer B.Cu) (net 9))
 (segment (start 80.645 85.725) (end 86.36 85.725) (width 0.7) (layer B.Cu) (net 9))
 (segment (start 86.36 85.725) (end 91.44 90.805) (width 0.7) (layer B.Cu) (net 9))
 (segment (start 131.804999 82.825001) (end 132.08 82.55) (width 0.7) (layer B.Cu) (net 10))
 (segment (start 126.015001 82.825001) (end 131.804999 82.825001) (width 0.7) (layer B.Cu) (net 10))
 (segment (start 132.08 78.105) (end 132.08 82.55) (width 0.7) (layer B.Cu) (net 10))
 (segment (start 136.525 73.66) (end 132.08 78.105) (width 0.7) (layer B.Cu) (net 10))
 (segment (start 139.62 70.565) (end 136.525 73.66) (width 0.7) (layer B.Cu) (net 10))
 (segment (start 132.08 62.23) (end 134.62 64.77) (width 0.7) (layer B.Cu) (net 10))
 (segment (start 132.08 59.055) (end 132.08 62.23) (width 0.7) (layer B.Cu) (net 10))
 (segment (start 151.05 70.565) (end 139.62 70.565) (width 0.7) (layer B.Cu) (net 10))
 (segment (start 134.62 64.77) (end 151.13 64.77) (width 0.7) (layer B.Cu) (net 10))
 (segment (start 151.13 64.77) (end 152.4 66.04) (width 0.7) (layer B.Cu) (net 10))
 (segment (start 152.4 66.04) (end 152.4 69.215) (width 0.7) (layer B.Cu) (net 10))
 (segment (start 152.4 69.215) (end 151.05 70.565) (width 0.7) (layer B.Cu) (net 10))
 (segment (start 84.455 92.075) (end 85.725 92.075) (width 0.7) (layer B.Cu) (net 11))
 (segment (start 80.645 88.265) (end 84.455 92.075) (width 0.7) (layer B.Cu) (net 11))
 (segment (start 85.09 92.075) (end 85.725 92.075) (width 0.7) (layer B.Cu) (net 11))
 (segment (start 109.975002 73.465) (end 110.775001 72.665001) (width 0.7) (layer B.Cu) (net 11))
 (segment (start 106.68 76.760002) (end 109.975002 73.465) (width 0.7) (layer B.Cu) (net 11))
 (segment (start 106.68 88.265) (end 106.68 76.760002) (width 0.7) (layer B.Cu) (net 11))
 (segment (start 85.725 92.075) (end 102.87 92.075) (width 0.7) (layer B.Cu) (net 11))
 (segment (start 102.87 92.075) (end 106.68 88.265) (width 0.7) (layer B.Cu) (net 11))
 (segment (start 78.74 72.39) (end 80.645 70.485) (width 0.7) (layer B.Cu) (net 13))
 (segment (start 78.74 90.17) (end 78.74 72.39) (width 0.7) (layer B.Cu) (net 13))
 (segment (start 81.915 93.345) (end 78.74 90.17) (width 0.7) (layer B.Cu) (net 13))
 (segment (start 113.305001 75.205001) (end 119.38 81.28) (width 0.7) (layer B.Cu) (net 13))
 (segment (start 110.775001 75.205001) (end 113.305001 75.205001) (width 0.7) (layer B.Cu) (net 13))
 (segment (start 119.38 81.28) (end 119.38 89.535) (width 0.7) (layer B.Cu) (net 13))
 (segment (start 119.38 89.535) (end 111.76 97.155) (width 0.7) (layer B.Cu) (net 13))
 (segment (start 111.76 97.155) (end 109.855 97.155) (width 0.7) (layer B.Cu) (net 13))
 (segment (start 109.855 97.155) (end 107.95 95.25) (width 0.7) (layer B.Cu) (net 13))
 (segment (start 107.95 95.25) (end 106.045 93.345) (width 0.7) (layer B.Cu) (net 13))
 (segment (start 106.045 93.345) (end 81.915 93.345) (width 0.7) (layer B.Cu) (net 13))
 (segment (start 110.775001 77.745001) (end 112.670001 77.745001) (width 0.7) (layer B.Cu) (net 15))
 (segment (start 112.670001 77.745001) (end 116.205 81.28) (width 0.7) (layer B.Cu) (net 15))
 (segment (start 116.205 81.28) (end 116.205 85.725) (width 0.7) (layer B.Cu) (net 15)))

